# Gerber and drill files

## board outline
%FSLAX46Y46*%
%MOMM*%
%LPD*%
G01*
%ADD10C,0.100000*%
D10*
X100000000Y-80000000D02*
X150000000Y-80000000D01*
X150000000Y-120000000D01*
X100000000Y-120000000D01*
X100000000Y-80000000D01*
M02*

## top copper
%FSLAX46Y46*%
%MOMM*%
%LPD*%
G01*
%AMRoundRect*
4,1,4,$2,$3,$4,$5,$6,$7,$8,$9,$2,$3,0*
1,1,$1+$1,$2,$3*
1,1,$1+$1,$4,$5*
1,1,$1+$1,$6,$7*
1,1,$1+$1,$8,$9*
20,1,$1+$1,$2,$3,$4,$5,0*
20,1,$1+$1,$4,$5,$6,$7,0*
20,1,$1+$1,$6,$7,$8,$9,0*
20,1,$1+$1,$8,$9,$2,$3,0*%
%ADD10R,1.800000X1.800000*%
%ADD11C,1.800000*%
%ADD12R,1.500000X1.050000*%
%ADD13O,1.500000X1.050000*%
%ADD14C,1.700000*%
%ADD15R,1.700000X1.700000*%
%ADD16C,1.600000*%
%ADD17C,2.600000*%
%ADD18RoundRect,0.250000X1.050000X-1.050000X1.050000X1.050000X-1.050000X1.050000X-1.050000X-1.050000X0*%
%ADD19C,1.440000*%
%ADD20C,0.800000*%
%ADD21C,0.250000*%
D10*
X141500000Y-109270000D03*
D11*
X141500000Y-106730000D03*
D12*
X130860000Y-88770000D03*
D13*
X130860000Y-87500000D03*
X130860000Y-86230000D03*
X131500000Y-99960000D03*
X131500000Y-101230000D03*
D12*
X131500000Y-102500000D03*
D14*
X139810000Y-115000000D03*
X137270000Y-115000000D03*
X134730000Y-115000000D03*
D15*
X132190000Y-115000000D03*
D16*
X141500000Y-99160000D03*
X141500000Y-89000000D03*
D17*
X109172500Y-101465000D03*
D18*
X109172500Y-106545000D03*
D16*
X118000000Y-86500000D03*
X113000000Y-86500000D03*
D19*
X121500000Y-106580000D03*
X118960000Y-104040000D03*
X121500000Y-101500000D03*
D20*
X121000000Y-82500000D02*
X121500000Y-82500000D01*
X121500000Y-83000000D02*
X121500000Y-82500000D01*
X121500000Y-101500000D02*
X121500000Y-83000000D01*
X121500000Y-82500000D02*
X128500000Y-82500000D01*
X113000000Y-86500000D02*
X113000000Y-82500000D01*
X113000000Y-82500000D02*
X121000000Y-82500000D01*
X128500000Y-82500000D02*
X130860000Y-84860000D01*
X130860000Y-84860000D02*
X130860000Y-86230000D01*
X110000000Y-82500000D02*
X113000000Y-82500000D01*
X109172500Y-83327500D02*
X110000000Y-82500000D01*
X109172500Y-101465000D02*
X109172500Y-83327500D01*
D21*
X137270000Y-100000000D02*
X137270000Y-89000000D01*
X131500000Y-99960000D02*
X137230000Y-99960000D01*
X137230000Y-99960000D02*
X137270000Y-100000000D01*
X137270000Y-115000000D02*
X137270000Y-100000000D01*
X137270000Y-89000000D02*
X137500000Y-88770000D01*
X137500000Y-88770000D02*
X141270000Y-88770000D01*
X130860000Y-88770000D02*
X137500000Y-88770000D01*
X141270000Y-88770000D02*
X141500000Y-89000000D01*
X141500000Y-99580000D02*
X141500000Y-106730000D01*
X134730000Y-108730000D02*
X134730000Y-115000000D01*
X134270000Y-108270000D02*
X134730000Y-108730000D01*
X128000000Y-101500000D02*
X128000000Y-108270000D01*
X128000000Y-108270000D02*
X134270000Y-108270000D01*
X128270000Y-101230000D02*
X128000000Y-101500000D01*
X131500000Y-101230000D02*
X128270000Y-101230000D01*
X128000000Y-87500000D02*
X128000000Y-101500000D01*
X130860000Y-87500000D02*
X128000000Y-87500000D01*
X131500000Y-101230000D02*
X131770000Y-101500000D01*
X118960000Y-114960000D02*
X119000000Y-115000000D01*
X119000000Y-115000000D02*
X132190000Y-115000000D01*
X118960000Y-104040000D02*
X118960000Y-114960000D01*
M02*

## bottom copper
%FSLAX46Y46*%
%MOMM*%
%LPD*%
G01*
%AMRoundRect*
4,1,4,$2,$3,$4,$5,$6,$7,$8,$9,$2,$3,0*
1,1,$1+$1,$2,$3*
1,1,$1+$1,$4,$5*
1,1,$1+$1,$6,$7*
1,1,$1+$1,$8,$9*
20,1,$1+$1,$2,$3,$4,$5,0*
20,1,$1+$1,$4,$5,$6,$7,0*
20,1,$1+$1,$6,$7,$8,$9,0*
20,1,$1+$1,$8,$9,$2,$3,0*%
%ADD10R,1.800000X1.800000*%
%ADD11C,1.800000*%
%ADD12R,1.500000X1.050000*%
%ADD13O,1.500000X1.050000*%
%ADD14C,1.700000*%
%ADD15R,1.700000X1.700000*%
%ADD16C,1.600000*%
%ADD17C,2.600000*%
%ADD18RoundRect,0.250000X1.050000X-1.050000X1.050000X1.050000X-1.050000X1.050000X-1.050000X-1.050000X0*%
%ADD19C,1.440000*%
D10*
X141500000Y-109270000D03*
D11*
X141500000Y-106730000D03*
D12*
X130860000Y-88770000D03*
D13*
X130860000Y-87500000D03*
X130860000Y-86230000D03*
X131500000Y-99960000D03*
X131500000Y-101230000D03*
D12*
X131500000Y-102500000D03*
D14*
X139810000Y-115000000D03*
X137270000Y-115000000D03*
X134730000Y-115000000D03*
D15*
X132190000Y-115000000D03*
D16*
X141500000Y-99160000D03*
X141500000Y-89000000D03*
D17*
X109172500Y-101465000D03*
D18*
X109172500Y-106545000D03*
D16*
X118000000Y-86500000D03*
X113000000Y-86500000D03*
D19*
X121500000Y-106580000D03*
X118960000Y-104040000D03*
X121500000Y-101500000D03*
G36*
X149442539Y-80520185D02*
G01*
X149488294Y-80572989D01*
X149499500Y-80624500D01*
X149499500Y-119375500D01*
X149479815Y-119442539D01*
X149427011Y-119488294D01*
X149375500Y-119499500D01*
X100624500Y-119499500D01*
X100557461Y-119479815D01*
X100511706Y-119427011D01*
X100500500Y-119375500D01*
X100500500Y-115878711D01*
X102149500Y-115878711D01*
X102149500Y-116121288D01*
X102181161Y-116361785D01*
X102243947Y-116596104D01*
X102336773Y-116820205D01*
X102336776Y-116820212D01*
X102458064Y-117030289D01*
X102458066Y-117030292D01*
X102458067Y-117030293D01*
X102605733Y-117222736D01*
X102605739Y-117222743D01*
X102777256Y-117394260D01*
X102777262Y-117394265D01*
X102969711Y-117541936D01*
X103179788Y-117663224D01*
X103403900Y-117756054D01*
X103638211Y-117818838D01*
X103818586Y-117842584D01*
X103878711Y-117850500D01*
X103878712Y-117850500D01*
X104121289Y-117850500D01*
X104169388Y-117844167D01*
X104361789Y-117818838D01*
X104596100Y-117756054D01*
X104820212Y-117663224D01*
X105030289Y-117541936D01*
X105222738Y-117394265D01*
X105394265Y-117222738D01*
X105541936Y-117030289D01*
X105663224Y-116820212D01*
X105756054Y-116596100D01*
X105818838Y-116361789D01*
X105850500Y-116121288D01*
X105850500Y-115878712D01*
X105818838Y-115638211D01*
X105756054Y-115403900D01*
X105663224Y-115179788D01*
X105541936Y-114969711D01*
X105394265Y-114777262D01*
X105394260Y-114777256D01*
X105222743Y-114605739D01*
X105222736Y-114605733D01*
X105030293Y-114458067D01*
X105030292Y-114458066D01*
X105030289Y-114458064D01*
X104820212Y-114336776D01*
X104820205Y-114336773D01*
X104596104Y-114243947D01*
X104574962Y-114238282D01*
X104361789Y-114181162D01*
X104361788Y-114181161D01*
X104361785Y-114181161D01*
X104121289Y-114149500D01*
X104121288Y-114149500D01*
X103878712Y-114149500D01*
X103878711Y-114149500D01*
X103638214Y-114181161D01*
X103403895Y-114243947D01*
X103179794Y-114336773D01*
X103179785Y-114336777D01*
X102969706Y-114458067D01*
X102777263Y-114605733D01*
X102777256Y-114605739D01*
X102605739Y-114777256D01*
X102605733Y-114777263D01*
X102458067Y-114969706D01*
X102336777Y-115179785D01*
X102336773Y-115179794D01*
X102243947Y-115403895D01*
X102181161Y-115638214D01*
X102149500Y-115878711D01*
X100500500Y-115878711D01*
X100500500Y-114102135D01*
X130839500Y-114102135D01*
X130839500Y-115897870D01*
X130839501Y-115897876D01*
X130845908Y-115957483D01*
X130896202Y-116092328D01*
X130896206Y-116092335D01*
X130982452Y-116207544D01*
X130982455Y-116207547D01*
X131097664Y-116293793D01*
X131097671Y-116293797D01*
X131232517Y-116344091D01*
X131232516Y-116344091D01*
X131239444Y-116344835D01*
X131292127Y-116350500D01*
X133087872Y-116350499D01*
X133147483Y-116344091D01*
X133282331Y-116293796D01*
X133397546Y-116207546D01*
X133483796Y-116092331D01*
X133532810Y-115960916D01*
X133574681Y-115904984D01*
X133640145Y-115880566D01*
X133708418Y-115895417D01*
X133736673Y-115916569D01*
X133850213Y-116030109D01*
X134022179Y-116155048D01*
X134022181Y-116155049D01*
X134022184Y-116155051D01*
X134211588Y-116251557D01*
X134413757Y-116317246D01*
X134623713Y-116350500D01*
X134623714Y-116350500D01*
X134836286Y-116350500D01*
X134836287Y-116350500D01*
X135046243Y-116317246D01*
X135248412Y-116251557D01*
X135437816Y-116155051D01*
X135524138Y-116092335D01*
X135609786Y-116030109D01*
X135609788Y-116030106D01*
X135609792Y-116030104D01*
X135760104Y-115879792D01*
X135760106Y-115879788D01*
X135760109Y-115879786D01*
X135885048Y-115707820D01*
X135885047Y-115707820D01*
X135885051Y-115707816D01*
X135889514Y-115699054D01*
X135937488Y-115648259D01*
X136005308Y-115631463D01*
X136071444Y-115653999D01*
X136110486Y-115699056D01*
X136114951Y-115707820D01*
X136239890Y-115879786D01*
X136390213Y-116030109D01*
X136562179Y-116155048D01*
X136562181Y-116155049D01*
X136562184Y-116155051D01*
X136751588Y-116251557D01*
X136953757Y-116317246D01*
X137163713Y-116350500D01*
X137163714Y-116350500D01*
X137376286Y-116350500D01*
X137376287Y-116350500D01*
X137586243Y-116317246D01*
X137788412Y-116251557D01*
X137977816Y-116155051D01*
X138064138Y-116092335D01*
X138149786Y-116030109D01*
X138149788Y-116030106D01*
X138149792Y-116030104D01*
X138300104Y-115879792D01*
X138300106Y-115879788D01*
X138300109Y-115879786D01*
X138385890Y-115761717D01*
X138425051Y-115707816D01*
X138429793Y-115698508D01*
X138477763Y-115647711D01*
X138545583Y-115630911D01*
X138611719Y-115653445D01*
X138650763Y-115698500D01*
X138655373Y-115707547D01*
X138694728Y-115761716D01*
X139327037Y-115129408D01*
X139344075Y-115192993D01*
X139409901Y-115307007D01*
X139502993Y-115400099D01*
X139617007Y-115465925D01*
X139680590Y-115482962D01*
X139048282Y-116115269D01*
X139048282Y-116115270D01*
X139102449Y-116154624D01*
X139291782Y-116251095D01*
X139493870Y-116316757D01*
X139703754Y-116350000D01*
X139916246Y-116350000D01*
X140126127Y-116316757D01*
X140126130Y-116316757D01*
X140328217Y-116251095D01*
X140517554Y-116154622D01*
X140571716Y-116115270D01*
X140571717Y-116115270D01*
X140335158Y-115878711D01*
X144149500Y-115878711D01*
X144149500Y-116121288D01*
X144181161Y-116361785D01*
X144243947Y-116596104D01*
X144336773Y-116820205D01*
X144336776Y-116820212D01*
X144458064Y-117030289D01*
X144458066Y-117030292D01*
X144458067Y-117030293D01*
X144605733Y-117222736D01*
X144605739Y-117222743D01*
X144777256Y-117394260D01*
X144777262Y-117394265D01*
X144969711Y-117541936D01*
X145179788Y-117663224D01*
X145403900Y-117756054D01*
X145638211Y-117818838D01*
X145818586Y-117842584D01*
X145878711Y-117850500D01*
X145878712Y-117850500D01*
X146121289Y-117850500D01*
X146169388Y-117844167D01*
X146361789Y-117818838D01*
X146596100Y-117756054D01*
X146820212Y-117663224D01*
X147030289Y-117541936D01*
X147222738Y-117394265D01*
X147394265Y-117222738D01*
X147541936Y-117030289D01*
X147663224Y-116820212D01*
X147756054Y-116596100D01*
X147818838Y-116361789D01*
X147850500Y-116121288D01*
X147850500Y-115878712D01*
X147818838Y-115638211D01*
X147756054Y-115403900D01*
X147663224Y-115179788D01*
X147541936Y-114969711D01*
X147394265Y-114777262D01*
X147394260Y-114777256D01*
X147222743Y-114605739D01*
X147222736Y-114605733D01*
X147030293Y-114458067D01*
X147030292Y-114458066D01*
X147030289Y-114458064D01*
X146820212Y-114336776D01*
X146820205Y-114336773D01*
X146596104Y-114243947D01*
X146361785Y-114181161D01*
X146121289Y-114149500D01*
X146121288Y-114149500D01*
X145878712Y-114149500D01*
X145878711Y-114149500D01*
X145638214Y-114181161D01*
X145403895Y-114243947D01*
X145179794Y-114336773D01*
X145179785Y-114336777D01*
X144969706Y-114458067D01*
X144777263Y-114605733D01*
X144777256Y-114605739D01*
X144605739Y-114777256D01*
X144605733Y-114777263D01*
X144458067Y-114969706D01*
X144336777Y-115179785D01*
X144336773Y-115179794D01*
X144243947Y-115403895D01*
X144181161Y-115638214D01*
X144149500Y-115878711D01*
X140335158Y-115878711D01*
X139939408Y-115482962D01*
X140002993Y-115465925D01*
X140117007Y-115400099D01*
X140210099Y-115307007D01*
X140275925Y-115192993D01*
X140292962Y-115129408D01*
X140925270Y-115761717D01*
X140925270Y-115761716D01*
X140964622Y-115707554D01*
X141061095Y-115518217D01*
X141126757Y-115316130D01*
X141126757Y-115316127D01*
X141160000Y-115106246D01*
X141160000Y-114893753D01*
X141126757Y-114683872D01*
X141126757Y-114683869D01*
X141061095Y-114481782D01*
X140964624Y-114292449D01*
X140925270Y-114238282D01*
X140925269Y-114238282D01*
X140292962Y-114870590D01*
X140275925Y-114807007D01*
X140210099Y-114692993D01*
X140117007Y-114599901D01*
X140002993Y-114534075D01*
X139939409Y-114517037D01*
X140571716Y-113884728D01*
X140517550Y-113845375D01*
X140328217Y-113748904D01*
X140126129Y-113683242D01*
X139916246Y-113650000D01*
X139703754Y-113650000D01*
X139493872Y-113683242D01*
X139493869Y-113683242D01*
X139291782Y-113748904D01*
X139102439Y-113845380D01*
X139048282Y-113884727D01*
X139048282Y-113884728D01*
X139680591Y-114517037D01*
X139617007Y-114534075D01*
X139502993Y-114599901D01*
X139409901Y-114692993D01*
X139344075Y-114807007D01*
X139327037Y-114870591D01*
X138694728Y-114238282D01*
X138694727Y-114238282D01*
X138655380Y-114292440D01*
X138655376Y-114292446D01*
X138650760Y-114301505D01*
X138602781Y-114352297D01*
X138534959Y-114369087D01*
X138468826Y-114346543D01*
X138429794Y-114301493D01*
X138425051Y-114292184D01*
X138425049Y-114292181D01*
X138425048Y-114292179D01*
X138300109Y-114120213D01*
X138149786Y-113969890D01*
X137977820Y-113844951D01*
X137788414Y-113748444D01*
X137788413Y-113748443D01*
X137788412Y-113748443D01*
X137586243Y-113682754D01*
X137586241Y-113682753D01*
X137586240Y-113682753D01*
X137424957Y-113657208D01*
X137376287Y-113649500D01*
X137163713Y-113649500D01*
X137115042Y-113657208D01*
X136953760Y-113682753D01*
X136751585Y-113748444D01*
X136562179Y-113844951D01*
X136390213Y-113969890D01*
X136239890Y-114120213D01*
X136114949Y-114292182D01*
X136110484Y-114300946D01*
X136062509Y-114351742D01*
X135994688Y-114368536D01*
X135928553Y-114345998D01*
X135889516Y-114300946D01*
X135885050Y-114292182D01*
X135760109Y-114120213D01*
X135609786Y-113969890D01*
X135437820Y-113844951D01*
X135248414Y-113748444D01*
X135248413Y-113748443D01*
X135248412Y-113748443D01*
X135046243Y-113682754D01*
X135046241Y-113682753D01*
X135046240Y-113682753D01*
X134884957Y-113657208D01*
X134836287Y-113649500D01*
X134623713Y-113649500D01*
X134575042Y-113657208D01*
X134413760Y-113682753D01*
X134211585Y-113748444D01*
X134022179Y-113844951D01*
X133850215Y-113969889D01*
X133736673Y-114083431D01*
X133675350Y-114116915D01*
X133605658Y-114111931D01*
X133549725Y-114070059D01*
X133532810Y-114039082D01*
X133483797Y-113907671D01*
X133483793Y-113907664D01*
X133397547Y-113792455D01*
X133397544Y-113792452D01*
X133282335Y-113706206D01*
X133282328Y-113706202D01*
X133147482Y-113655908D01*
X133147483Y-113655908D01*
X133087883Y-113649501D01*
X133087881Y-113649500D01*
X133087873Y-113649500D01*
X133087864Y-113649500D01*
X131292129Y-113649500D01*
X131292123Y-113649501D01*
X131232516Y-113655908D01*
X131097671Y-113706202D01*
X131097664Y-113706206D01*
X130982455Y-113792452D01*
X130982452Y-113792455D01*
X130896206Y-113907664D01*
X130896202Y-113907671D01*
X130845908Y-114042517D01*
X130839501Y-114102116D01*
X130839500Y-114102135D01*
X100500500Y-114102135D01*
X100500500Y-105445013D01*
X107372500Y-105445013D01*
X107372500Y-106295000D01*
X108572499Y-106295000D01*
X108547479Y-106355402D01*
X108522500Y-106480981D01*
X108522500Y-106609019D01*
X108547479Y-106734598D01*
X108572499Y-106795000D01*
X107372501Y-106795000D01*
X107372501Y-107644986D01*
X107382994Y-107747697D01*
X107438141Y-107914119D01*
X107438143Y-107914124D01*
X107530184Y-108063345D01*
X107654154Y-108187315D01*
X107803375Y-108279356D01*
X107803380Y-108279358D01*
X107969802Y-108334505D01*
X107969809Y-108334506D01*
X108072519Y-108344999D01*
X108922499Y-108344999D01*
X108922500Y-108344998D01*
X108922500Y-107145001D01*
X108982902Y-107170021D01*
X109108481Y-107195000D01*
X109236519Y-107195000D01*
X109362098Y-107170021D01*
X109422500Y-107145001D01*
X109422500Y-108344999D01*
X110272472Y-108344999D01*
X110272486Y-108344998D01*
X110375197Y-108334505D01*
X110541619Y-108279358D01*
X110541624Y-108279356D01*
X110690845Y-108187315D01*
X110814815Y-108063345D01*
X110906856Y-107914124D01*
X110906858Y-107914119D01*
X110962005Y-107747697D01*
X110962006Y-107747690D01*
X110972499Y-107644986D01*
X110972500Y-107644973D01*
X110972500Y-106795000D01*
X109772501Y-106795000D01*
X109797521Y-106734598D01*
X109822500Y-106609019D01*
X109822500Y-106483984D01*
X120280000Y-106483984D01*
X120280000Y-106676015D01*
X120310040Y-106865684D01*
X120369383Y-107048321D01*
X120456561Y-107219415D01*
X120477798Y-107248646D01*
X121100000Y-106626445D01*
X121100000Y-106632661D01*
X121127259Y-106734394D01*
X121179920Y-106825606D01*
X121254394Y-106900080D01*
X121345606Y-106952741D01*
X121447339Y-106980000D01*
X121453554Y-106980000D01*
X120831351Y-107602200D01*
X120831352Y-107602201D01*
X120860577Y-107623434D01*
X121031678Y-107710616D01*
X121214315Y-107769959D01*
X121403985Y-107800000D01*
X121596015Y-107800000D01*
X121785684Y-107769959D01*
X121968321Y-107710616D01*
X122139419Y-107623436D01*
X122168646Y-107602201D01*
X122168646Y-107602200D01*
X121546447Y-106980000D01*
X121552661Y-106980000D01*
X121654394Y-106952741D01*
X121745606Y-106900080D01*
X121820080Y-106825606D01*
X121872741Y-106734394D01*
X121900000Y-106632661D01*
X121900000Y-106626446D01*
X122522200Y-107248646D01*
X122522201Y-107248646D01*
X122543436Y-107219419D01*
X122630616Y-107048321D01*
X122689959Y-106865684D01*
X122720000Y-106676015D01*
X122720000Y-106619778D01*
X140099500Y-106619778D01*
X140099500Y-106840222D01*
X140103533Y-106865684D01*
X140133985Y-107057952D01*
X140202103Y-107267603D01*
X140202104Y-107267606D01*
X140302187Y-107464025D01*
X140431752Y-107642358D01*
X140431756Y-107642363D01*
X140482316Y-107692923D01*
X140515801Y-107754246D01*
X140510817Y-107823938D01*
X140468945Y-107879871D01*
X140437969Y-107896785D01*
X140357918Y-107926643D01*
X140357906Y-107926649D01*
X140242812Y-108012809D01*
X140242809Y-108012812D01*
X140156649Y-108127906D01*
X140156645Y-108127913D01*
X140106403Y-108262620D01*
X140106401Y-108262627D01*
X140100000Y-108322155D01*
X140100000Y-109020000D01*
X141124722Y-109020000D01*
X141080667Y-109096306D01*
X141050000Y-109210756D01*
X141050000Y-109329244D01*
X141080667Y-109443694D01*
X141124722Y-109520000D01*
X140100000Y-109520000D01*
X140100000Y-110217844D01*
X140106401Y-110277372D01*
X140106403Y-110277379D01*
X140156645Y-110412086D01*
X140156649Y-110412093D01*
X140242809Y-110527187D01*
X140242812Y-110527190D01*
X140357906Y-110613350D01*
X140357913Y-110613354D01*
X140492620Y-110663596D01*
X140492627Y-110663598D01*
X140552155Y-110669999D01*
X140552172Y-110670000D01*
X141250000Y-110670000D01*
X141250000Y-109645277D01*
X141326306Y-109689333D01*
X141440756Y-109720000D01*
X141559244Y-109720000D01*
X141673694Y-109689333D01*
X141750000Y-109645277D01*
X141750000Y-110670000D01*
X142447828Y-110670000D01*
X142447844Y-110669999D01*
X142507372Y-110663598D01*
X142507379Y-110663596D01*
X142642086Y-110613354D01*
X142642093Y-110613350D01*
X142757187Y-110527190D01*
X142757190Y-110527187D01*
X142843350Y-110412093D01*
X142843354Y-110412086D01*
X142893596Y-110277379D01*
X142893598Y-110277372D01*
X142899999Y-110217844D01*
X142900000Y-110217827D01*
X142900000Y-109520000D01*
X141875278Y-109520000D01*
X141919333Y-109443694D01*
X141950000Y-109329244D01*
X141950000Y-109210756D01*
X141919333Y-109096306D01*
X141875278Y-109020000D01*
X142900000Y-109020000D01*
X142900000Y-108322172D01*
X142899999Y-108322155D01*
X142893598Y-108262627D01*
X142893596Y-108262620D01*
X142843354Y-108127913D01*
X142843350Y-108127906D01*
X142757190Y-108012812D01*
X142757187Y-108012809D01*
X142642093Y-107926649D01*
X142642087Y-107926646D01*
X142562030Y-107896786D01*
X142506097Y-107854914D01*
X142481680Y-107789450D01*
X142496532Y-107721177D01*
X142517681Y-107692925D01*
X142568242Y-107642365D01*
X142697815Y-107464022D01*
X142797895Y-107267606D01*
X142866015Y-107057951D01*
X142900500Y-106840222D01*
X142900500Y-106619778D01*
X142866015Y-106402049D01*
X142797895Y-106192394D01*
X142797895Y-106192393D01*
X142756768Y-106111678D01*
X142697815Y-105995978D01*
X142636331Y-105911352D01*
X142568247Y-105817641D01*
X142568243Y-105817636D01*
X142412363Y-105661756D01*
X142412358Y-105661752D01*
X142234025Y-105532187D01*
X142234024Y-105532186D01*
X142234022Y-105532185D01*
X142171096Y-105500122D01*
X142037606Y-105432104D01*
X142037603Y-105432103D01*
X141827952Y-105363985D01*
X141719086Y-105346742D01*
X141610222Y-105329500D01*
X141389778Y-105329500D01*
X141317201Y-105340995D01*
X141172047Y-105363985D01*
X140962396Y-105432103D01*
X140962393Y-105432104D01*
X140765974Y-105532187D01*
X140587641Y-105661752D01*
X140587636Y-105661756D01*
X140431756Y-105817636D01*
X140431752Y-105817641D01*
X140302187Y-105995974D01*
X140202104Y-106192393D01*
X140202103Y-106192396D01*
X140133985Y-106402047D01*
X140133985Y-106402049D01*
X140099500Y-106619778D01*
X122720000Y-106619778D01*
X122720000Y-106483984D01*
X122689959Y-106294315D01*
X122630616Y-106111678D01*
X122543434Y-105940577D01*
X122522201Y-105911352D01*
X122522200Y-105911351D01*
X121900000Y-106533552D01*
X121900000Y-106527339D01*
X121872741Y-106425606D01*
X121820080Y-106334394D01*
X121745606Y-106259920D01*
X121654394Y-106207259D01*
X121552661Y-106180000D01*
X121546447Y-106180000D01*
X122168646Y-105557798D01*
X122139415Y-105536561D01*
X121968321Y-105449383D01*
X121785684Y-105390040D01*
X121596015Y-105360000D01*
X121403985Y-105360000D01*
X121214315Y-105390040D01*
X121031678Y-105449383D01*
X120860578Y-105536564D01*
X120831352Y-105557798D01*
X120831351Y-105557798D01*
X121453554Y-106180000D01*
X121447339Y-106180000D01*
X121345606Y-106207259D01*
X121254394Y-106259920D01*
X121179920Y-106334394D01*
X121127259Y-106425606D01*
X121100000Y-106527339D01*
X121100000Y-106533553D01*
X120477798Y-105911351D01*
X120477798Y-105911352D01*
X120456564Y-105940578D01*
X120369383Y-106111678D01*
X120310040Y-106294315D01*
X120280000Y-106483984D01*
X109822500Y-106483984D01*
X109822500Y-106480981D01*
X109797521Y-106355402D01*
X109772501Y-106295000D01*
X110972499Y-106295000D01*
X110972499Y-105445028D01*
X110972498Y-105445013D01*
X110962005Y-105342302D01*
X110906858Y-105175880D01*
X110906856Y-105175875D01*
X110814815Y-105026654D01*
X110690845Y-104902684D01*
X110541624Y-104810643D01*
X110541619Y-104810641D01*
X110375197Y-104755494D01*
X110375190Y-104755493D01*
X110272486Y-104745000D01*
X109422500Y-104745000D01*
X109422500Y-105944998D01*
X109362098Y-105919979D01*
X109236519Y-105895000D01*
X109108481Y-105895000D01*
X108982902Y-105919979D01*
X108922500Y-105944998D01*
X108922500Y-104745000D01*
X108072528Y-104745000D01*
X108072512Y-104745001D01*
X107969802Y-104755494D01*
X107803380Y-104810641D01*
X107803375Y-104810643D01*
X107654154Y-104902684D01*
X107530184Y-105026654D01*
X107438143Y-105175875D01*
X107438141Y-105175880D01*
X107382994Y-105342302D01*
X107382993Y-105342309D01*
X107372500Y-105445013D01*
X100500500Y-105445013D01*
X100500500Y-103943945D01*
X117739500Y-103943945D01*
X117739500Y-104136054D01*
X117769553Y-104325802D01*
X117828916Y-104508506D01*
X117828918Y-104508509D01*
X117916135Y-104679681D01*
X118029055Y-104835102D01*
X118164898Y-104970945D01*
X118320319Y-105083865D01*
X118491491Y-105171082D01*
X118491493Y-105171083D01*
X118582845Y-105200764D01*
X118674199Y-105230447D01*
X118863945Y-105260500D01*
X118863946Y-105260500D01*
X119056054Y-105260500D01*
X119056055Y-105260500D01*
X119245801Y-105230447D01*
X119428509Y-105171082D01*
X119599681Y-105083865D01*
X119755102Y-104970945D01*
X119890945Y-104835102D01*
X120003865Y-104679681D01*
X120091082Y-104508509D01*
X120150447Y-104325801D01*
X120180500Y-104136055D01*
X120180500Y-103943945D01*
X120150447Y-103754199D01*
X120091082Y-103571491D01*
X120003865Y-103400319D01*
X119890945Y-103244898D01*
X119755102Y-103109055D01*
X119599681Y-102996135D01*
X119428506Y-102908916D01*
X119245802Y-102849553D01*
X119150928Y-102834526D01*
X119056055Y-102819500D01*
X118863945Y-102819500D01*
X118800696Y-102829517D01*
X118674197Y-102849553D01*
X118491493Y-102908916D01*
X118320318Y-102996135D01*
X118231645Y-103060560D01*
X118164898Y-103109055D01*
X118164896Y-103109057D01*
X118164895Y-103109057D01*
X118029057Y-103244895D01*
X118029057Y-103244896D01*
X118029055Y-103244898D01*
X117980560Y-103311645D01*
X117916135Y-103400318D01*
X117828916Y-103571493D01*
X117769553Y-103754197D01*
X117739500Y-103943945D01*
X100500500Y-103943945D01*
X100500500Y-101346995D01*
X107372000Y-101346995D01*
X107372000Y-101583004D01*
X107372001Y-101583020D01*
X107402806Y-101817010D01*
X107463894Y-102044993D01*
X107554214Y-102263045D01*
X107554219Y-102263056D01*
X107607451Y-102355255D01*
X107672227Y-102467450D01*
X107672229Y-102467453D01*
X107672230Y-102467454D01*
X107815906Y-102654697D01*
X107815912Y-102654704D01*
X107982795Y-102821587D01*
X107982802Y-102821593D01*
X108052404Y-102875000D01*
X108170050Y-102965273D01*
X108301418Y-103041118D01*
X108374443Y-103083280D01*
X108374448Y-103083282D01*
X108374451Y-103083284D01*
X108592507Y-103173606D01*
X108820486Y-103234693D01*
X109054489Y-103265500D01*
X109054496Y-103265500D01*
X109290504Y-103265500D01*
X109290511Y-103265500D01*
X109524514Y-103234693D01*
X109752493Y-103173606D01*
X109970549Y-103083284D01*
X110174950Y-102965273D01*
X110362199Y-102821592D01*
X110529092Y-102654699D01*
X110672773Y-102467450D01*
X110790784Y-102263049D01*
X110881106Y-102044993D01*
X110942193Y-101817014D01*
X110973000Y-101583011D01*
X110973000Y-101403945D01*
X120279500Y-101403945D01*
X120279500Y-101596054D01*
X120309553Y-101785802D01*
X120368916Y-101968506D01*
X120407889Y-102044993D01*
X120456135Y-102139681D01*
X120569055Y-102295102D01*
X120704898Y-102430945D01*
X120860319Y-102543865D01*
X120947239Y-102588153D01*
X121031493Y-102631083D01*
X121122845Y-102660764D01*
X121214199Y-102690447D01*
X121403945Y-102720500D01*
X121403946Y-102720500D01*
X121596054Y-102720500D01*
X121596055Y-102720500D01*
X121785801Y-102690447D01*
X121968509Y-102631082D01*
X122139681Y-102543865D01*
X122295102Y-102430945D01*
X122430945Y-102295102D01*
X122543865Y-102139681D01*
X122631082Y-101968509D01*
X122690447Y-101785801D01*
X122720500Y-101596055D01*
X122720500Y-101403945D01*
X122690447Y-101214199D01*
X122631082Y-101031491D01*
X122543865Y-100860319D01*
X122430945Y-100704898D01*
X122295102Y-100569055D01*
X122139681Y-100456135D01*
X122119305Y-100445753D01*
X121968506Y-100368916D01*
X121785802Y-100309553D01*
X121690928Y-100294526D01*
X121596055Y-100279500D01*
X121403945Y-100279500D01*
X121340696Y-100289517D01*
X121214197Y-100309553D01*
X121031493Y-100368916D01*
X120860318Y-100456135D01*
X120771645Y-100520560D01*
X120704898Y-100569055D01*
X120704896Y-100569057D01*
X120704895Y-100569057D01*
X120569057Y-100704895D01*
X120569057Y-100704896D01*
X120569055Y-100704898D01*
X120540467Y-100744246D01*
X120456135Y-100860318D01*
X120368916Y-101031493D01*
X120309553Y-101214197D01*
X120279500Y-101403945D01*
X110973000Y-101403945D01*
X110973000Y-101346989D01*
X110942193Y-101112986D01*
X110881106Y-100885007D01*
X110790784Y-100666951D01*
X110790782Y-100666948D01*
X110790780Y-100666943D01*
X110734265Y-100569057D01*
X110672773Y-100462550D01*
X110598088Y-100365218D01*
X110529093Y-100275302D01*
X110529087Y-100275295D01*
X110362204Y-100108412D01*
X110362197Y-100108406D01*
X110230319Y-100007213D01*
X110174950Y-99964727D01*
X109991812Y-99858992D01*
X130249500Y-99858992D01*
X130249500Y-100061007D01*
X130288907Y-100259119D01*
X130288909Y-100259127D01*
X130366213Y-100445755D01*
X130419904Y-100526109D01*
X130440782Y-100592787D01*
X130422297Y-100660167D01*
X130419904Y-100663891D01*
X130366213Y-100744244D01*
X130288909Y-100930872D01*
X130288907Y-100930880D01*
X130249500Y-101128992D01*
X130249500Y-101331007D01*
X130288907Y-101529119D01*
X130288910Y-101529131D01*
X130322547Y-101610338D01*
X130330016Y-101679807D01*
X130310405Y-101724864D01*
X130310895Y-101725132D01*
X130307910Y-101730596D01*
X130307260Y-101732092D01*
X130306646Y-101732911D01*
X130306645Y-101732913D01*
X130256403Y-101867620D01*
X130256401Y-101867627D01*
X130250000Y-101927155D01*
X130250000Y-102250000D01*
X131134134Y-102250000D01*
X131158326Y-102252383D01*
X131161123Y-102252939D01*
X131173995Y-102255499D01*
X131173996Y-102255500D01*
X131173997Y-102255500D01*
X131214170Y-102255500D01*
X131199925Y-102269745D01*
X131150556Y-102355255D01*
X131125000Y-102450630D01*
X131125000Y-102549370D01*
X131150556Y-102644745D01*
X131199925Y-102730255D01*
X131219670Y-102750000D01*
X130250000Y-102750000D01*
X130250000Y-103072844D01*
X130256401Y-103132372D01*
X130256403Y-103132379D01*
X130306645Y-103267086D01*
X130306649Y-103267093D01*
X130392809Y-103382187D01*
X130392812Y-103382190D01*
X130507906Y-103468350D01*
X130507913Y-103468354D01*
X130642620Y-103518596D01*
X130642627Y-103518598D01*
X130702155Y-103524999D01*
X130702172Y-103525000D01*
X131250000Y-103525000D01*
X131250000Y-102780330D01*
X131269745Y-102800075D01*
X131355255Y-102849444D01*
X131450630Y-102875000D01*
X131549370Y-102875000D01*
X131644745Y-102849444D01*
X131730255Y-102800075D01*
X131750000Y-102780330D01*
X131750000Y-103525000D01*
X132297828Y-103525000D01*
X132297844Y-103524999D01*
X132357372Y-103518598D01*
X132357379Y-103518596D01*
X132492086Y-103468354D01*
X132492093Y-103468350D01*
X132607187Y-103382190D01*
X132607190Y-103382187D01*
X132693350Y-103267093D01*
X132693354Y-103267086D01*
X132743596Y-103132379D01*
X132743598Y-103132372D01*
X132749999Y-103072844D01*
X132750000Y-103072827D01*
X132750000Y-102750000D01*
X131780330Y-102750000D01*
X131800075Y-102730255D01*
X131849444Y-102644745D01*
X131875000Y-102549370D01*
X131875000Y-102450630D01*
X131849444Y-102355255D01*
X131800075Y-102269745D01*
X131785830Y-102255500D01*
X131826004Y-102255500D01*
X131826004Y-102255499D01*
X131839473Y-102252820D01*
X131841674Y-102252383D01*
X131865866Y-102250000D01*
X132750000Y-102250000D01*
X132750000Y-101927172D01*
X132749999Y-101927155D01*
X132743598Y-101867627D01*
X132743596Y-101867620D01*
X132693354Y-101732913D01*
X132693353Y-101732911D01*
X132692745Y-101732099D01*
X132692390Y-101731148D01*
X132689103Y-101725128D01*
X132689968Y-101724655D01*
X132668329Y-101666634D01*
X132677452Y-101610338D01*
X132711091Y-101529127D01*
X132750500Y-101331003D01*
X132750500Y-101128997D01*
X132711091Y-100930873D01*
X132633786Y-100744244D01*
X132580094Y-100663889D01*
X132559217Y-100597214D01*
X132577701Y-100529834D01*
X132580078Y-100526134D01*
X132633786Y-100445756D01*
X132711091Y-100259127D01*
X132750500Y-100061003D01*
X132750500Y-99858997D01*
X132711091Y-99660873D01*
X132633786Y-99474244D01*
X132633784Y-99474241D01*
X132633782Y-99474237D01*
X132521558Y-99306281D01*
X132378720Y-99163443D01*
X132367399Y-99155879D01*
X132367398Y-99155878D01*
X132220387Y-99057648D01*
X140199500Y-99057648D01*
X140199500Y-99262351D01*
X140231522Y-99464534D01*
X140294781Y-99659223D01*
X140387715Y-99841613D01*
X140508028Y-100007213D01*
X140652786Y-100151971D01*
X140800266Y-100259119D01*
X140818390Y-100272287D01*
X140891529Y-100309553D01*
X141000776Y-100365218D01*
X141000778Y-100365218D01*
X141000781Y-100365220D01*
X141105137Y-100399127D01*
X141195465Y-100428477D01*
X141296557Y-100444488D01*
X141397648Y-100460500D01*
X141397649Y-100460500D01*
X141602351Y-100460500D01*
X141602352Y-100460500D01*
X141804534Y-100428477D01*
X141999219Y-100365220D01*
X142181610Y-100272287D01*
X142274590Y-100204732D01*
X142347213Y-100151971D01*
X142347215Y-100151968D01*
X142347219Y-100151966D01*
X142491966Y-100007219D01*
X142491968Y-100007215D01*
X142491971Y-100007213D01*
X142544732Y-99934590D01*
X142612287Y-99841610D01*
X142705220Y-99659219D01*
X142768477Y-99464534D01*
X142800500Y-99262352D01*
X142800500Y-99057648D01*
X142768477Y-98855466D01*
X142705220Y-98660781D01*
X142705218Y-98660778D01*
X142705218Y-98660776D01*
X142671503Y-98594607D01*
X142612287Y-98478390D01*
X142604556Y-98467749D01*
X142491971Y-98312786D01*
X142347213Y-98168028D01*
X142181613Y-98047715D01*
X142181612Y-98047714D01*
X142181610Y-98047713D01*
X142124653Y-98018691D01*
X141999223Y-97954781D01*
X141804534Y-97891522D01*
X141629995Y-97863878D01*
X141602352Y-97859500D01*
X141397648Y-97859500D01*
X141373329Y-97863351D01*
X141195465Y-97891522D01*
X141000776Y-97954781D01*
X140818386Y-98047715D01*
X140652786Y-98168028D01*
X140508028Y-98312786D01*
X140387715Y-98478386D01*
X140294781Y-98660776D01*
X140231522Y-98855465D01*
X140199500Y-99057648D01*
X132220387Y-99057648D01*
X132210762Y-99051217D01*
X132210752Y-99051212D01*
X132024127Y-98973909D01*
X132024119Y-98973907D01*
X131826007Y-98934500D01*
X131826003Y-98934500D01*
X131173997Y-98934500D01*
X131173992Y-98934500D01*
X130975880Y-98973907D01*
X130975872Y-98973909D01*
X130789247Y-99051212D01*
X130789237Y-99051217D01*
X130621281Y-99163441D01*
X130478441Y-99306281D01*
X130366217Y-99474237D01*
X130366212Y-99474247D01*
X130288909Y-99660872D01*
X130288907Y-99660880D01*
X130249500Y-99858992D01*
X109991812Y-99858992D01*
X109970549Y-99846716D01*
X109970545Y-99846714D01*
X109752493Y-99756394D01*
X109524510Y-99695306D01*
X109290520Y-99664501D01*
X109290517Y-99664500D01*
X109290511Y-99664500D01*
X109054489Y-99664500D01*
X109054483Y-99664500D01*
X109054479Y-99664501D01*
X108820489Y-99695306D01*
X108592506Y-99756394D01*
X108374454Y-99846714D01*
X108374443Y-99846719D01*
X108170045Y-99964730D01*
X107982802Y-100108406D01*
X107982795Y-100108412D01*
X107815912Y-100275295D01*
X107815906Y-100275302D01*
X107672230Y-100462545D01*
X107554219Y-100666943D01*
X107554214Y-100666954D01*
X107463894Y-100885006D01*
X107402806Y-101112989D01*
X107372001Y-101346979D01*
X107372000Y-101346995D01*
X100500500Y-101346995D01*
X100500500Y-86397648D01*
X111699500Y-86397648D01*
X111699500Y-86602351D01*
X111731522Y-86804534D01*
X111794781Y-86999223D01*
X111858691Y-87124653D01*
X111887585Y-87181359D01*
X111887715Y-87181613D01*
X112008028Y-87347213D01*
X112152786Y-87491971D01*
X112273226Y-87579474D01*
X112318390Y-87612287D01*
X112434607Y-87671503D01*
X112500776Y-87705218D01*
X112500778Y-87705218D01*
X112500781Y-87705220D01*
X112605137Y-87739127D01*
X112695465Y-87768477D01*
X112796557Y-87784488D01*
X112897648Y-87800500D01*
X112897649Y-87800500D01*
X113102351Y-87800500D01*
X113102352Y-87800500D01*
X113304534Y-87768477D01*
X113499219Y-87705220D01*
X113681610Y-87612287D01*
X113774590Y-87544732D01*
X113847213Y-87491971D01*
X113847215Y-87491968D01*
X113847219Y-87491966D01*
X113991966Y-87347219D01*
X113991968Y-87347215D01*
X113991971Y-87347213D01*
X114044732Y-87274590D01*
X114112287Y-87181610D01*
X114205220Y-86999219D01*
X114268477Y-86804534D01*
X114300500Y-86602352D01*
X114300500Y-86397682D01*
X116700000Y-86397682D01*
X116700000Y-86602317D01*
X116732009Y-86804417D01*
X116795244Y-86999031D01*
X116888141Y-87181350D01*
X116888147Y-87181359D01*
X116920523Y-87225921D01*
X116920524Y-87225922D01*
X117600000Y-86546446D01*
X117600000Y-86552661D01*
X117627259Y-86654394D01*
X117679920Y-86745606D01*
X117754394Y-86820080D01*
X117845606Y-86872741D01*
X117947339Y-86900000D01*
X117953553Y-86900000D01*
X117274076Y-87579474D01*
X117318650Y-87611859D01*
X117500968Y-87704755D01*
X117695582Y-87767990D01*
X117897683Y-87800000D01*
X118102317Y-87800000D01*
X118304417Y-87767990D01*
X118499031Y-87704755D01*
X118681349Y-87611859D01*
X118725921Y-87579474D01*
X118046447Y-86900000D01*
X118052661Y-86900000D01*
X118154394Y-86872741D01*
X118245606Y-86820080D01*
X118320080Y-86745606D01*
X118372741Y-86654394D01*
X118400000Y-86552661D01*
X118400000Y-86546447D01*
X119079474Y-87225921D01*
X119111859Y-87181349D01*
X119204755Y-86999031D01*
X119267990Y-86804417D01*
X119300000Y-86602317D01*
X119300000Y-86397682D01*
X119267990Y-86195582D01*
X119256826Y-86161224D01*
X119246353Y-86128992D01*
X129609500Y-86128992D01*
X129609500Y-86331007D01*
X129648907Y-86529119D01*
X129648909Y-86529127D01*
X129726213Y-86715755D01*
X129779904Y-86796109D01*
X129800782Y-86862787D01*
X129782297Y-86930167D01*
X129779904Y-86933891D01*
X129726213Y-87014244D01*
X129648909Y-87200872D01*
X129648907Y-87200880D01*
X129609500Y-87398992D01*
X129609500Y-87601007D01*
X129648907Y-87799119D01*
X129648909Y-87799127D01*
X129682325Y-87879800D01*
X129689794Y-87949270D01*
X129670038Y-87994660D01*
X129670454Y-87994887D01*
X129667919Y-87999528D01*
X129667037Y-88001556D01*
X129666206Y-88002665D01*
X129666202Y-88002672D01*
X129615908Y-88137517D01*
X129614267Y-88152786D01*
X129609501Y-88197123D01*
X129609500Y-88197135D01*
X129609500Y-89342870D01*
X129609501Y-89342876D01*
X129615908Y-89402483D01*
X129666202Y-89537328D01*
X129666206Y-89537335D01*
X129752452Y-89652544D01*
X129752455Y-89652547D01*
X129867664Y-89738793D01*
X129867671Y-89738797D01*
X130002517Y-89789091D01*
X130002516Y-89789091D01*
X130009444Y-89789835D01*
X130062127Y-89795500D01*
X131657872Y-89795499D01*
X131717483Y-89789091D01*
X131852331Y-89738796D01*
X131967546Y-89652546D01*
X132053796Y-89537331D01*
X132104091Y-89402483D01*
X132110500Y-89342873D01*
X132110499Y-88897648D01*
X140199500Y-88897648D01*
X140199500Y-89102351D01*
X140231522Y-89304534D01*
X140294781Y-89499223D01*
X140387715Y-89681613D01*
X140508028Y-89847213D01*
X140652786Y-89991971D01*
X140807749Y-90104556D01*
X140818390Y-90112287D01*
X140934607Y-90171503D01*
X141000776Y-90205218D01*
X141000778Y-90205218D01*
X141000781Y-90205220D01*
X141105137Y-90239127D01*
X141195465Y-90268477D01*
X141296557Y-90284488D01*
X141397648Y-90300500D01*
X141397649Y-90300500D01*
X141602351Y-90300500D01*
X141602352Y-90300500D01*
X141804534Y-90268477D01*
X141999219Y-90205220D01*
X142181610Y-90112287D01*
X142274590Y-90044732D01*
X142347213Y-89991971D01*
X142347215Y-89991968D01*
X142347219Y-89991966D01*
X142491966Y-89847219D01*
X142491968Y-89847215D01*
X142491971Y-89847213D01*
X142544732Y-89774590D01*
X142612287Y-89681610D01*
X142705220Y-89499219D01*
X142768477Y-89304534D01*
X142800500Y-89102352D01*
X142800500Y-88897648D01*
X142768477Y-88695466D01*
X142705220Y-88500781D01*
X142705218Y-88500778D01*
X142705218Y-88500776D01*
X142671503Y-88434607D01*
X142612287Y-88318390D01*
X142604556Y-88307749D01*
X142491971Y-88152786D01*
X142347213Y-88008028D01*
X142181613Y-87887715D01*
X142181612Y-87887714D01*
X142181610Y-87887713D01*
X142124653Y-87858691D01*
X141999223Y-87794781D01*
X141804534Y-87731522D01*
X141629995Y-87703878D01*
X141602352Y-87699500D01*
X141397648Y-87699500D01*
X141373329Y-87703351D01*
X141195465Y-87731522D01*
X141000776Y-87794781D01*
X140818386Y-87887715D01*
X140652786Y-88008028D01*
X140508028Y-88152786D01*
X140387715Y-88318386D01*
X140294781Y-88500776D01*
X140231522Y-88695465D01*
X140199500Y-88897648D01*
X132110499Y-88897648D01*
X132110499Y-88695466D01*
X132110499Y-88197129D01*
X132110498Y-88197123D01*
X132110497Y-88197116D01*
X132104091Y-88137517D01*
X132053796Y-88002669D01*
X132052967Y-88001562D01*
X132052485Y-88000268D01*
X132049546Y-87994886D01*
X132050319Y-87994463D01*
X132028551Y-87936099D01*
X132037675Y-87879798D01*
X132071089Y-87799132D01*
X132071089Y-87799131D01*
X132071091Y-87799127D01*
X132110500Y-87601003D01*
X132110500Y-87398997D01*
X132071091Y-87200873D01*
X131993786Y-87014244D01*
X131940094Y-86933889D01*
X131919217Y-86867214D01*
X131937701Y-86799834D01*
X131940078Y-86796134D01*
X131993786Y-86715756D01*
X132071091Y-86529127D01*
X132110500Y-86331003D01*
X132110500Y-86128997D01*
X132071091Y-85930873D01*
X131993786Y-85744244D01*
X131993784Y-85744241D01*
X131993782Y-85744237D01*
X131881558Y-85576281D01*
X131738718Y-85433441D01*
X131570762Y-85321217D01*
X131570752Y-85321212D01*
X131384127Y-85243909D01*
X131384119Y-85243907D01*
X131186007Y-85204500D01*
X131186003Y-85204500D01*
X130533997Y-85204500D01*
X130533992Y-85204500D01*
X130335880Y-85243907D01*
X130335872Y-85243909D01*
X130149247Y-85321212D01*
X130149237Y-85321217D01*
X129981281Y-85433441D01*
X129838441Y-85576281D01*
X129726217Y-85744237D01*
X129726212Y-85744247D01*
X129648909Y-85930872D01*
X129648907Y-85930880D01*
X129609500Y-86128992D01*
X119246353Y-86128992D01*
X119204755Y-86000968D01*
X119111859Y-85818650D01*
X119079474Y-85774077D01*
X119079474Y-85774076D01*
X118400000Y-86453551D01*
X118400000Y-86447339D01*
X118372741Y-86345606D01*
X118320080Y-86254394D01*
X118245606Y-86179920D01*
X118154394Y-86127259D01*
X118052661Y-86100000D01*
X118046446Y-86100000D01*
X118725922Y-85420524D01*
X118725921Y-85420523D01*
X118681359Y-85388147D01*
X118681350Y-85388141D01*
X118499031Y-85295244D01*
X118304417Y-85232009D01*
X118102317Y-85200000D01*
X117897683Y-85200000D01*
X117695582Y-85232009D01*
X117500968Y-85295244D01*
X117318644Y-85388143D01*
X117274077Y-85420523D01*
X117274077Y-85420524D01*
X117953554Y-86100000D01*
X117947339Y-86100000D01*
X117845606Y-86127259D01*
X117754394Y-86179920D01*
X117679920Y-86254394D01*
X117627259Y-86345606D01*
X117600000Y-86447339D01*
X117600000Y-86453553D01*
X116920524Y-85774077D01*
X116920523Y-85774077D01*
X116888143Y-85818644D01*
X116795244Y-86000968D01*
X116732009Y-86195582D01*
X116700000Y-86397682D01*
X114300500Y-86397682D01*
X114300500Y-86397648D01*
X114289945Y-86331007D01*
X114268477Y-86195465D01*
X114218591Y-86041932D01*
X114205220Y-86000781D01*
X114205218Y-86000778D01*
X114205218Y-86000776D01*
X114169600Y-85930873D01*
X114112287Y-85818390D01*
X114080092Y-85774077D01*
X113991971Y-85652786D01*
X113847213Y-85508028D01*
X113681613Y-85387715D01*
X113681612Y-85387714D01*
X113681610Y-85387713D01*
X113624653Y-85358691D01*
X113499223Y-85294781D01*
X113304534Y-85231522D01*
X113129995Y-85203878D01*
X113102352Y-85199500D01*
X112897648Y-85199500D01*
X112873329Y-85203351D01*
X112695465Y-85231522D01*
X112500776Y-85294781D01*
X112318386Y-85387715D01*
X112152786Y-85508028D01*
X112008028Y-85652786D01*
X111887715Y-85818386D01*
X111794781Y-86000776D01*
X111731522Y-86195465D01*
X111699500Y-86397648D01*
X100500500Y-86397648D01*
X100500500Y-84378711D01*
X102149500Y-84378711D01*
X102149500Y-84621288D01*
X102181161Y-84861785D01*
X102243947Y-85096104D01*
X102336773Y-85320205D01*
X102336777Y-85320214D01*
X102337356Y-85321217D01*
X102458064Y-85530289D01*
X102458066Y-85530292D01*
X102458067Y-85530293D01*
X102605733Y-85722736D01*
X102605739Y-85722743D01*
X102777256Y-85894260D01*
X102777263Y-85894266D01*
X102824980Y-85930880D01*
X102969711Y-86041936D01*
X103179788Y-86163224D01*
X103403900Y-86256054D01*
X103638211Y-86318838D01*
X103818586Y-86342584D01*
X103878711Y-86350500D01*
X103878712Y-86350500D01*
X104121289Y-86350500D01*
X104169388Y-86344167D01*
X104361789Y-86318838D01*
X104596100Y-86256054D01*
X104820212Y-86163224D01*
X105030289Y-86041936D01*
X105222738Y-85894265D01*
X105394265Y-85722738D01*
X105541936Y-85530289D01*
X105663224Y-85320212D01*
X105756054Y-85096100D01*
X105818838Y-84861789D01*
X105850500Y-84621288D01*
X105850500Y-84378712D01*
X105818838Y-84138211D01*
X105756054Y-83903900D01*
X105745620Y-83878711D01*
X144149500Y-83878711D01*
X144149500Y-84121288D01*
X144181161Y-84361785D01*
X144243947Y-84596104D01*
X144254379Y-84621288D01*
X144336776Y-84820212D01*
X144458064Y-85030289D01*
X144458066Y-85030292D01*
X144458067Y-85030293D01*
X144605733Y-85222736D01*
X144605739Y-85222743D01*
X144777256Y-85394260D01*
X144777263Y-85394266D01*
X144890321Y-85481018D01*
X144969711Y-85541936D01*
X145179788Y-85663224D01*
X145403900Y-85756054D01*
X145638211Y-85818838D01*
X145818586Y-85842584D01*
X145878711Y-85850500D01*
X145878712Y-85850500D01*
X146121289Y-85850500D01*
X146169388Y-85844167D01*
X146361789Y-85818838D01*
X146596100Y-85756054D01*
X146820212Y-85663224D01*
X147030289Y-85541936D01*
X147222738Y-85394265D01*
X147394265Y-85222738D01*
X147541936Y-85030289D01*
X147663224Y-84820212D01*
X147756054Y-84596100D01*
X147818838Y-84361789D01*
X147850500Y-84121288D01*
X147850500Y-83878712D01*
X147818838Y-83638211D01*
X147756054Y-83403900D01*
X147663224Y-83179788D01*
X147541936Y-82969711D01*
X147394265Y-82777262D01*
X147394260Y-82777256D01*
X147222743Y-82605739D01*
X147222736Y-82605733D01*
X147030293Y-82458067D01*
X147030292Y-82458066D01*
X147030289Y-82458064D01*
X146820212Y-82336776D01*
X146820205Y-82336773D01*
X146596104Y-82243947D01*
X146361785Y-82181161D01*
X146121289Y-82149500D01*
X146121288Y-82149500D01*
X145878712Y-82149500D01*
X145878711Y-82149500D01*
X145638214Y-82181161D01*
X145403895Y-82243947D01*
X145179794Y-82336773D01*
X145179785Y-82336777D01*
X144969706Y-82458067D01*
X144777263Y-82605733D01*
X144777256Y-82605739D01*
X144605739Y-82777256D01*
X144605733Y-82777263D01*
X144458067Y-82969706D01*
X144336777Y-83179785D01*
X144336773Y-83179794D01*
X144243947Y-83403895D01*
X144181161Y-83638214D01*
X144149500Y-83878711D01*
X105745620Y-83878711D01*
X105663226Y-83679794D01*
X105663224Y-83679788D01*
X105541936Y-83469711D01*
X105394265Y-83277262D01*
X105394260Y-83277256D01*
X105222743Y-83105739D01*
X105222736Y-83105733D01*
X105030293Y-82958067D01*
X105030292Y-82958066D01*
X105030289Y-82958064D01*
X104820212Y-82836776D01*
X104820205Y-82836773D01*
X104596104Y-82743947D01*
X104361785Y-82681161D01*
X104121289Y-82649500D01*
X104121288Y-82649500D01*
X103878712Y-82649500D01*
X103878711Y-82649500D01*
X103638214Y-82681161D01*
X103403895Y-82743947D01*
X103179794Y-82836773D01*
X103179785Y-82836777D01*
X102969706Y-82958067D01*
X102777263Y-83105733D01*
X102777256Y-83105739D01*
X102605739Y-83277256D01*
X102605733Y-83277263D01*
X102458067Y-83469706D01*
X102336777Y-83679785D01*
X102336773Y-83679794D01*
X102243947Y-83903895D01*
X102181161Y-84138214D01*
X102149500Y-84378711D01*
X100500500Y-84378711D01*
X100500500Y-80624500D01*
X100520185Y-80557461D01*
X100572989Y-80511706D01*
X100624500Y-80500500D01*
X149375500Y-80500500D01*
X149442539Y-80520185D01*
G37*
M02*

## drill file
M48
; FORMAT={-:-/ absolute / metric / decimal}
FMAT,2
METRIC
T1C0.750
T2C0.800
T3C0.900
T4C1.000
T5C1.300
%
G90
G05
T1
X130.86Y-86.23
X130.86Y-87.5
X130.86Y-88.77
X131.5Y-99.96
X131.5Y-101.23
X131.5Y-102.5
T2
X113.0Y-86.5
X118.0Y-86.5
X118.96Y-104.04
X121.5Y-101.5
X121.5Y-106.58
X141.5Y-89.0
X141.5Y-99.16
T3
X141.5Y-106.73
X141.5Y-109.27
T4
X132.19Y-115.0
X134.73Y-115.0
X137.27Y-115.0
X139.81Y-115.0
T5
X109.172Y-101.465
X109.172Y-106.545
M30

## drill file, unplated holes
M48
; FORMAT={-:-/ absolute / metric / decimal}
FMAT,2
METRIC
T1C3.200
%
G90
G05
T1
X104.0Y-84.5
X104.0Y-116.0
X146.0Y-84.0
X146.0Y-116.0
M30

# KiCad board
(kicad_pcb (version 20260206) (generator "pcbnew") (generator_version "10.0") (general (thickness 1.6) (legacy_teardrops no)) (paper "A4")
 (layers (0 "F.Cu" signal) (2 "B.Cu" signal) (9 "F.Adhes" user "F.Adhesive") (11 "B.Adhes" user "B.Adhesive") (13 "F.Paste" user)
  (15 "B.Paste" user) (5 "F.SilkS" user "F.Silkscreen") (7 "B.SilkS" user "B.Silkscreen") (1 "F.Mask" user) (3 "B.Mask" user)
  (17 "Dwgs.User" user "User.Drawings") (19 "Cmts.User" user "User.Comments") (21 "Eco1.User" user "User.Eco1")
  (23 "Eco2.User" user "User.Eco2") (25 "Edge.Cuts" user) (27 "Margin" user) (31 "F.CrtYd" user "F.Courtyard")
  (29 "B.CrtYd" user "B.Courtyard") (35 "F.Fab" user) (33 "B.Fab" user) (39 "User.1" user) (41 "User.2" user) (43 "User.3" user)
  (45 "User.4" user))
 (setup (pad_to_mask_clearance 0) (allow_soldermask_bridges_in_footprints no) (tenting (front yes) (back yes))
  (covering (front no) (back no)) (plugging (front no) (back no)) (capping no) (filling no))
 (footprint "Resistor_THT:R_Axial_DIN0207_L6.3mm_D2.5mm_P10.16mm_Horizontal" (layer "F.Cu") (at 141.5 89 -90)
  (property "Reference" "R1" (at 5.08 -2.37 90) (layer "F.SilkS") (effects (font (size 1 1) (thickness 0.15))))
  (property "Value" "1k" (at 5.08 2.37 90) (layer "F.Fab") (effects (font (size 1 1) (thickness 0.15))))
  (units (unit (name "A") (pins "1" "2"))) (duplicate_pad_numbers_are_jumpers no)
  (pad "1" thru_hole circle (at 0 0 270) (size 1.6 1.6) (drill 0.8) (layers "*.Cu" "*.Mask") (remove_unused_layers no) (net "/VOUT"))
  (pad "2" thru_hole circle (at 10.16 0 270) (size 1.6 1.6) (drill 0.8) (layers "*.Cu" "*.Mask") (remove_unused_layers no)
   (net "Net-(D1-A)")))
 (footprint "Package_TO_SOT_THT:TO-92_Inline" (layer "F.Cu") (at 131.5 102.5 90)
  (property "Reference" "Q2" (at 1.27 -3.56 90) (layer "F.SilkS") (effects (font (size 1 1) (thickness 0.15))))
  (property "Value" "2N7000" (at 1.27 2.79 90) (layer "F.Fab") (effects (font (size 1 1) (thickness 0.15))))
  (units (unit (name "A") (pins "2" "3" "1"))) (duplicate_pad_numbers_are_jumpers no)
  (pad "1" thru_hole rect (at 0 0 90) (size 1.05 1.5) (drill 0.75) (layers "*.Cu" "*.Mask") (remove_unused_layers no) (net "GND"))
  (pad "2" thru_hole oval (at 1.27 0 90) (size 1.05 1.5) (drill 0.75) (layers "*.Cu" "*.Mask") (remove_unused_layers no) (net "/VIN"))
  (pad "3" thru_hole oval (at 2.54 0 90) (size 1.05 1.5) (drill 0.75) (layers "*.Cu" "*.Mask") (remove_unused_layers no) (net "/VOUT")))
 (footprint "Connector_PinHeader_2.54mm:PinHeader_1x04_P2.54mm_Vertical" (layer "F.Cu") (at 132.19 115 90)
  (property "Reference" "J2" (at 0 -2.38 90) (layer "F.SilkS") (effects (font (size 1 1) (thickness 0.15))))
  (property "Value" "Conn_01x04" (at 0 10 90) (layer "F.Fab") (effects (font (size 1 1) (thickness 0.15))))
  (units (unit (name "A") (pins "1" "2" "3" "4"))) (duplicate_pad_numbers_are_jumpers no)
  (pad "1" thru_hole rect (at 0 0 90) (size 1.7 1.7) (drill 1) (layers "*.Cu" "*.Mask") (remove_unused_layers no) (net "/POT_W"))
  (pad "2" thru_hole circle (at 0 2.54 90) (size 1.7 1.7) (drill 1) (layers "*.Cu" "*.Mask") (remove_unused_layers no) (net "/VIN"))
  (pad "3" thru_hole circle (at 0 5.08 90) (size 1.7 1.7) (drill 1) (layers "*.Cu" "*.Mask") (remove_unused_layers no) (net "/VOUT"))
  (pad "4" thru_hole circle (at 0 7.62 90) (size 1.7 1.7) (drill 1) (layers "*.Cu" "*.Mask") (remove_unused_layers no) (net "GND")))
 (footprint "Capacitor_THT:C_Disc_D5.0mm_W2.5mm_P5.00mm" (layer "F.Cu") (at 113 86.5)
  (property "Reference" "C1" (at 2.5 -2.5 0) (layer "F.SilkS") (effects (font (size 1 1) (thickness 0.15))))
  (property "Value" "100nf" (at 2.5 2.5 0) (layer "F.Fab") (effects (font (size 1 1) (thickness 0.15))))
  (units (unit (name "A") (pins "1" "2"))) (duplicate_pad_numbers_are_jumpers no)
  (pad "1" thru_hole circle (at 0 0) (size 1.6 1.6) (drill 0.8) (layers "*.Cu" "*.Mask") (remove_unused_layers no) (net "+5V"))
  (pad "2" thru_hole circle (at 5 0) (size 1.6 1.6) (drill 0.8) (layers "*.Cu" "*.Mask") (remove_unused_layers no) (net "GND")))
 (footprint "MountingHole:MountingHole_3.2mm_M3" (layer "F.Cu") (at 146 116)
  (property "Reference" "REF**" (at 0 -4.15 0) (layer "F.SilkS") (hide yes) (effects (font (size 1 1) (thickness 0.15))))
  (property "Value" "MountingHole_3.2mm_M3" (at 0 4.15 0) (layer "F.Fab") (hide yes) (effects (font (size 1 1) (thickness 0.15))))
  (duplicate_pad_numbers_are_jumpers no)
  (pad "" np_thru_hole circle (at 0 0) (size 3.2 3.2) (drill 3.2) (layers "*.Cu" "*.Mask")))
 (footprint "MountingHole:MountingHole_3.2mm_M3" (layer "F.Cu") (at 104 84.5)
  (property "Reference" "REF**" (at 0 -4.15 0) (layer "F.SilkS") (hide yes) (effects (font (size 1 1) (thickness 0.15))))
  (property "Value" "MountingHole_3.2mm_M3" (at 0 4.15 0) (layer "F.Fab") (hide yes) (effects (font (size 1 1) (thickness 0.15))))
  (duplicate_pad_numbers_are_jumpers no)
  (pad "" np_thru_hole circle (at 0 0) (size 3.2 3.2) (drill 3.2) (layers "*.Cu" "*.Mask")))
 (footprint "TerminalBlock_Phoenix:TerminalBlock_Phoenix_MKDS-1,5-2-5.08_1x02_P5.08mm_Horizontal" (layer "F.Cu") (at 109.1725 106.545 90)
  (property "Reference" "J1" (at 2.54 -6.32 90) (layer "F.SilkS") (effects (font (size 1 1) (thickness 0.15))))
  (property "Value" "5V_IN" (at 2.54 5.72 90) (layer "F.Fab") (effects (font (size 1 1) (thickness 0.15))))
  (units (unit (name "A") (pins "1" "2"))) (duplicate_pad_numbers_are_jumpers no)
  (pad "1" thru_hole roundrect (at 0 0 90) (size 2.6 2.6) (drill 1.3) (layers "*.Cu" "*.Mask") (remove_unused_layers no)
   (roundrect_rratio 0.096154) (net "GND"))
  (pad "2" thru_hole circle (at 5.08 0 90) (size 2.6 2.6) (drill 1.3) (layers "*.Cu" "*.Mask") (remove_unused_layers no) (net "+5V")))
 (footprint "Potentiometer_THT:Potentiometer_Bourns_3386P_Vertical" (layer "F.Cu") (at 121.5 101.5 180)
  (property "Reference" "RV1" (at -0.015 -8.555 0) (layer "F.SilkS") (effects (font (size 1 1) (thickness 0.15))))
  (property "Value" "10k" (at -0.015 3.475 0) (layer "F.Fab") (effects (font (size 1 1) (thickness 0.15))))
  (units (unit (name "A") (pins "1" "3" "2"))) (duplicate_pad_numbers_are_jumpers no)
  (pad "1" thru_hole circle (at 0 0 180) (size 1.44 1.44) (drill 0.8) (layers "*.Cu" "*.Mask") (remove_unused_layers no) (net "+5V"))
  (pad "2" thru_hole circle (at 2.54 -2.54 180) (size 1.44 1.44) (drill 0.8) (layers "*.Cu" "*.Mask") (remove_unused_layers no)
   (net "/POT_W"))
  (pad "3" thru_hole circle (at 0 -5.08 180) (size 1.44 1.44) (drill 0.8) (layers "*.Cu" "*.Mask") (remove_unused_layers no) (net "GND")))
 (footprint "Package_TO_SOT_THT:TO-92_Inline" (layer "F.Cu") (at 130.86 88.77 90)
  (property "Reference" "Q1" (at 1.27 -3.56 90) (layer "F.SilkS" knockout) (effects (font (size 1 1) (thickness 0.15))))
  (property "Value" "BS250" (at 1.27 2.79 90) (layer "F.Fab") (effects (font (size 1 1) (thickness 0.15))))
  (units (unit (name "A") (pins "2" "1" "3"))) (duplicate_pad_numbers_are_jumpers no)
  (pad "1" thru_hole rect (at 0 0 90) (size 1.05 1.5) (drill 0.75) (layers "*.Cu" "*.Mask") (remove_unused_layers no) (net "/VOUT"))
  (pad "2" thru_hole oval (at 1.27 0 90) (size 1.05 1.5) (drill 0.75) (layers "*.Cu" "*.Mask") (remove_unused_layers no) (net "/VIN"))
  (pad "3" thru_hole oval (at 2.54 0 90) (size 1.05 1.5) (drill 0.75) (layers "*.Cu" "*.Mask") (remove_unused_layers no) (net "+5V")))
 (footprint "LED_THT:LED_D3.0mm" (layer "F.Cu") (at 141.5 109.27 90)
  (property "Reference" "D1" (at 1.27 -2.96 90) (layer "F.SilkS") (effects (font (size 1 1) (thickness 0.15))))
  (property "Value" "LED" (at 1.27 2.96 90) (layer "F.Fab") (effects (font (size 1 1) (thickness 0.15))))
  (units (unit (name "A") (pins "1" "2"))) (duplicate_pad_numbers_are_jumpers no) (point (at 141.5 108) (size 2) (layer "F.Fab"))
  (pad "1" thru_hole rect (at 0 0 90) (size 1.8 1.8) (drill 0.9) (layers "*.Cu" "*.Mask") (remove_unused_layers no) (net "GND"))
  (pad "2" thru_hole circle (at 2.54 0 90) (size 1.8 1.8) (drill 0.9) (layers "*.Cu" "*.Mask") (remove_unused_layers no) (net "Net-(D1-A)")))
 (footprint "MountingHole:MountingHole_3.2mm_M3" (layer "F.Cu") (at 146 84)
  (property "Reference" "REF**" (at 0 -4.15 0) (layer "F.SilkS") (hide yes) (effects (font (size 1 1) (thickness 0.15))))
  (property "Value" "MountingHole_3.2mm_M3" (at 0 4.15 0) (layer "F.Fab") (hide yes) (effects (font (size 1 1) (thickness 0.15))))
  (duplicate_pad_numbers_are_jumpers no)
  (pad "" np_thru_hole circle (at 0 0) (size 3.2 3.2) (drill 3.2) (layers "*.Cu" "*.Mask")))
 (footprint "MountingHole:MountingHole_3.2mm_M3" (layer "F.Cu") (at 104 116)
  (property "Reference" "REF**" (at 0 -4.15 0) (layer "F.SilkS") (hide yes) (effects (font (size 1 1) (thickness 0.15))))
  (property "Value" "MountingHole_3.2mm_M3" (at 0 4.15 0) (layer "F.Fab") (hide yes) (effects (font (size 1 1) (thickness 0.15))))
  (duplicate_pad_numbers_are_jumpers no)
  (pad "" np_thru_hole circle (at 0 0) (size 3.2 3.2) (drill 3.2) (layers "*.Cu" "*.Mask")))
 (gr_rect (start 100 80) (end 150 120) (stroke (width 0.1) (type default)) (fill no) (layer "Edge.Cuts"))
 (segment (start 137.23 99.96) (end 137.27 100) (width 0.25) (layer "F.Cu") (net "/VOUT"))
 (segment (start 131.5 99.96) (end 137.23 99.96) (width 0.25) (layer "F.Cu") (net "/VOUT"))
 (segment (start 137.5 88.77) (end 141.27 88.77) (width 0.25) (layer "F.Cu") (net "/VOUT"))
 (segment (start 130.86 88.77) (end 137.5 88.77) (width 0.25) (layer "F.Cu") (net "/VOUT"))
 (segment (start 137.27 115) (end 137.27 100) (width 0.25) (layer "F.Cu") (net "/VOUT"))
 (segment (start 141.27 88.77) (end 141.5 89) (width 0.25) (layer "F.Cu") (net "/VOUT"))
 (segment (start 137.27 100) (end 137.27 89) (width 0.25) (layer "F.Cu") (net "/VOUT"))
 (segment (start 137.27 89) (end 137.5 88.77) (width 0.25) (layer "F.Cu") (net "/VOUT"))
 (segment (start 141.5 99.58) (end 141.5 106.73) (width 0.25) (layer "F.Cu") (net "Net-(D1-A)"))
 (segment (start 128 87.5) (end 128 101.5) (width 0.25) (layer "F.Cu") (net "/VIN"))
 (segment (start 131.5 101.23) (end 131.77 101.5) (width 0.25) (layer "F.Cu") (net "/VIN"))
 (segment (start 134.27 108.27) (end 134.73 108.73) (width 0.25) (layer "F.Cu") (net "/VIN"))
 (segment (start 128.27 101.23) (end 128 101.5) (width 0.25) (layer "F.Cu") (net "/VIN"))
 (segment (start 128 101.5) (end 128 108.27) (width 0.25) (layer "F.Cu") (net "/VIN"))
 (segment (start 131.5 101.23) (end 128.27 101.23) (width 0.25) (layer "F.Cu") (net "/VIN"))
 (segment (start 134.73 108.73) (end 134.73 115) (width 0.25) (layer "F.Cu") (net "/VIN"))
 (segment (start 130.86 87.5) (end 128 87.5) (width 0.25) (layer "F.Cu") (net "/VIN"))
 (segment (start 128 108.27) (end 134.27 108.27) (width 0.25) (layer "F.Cu") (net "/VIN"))
 (segment (start 118.96 104.04) (end 118.96 114.96) (width 0.25) (layer "F.Cu") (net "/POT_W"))
 (segment (start 118.96 114.96) (end 119 115) (width 0.25) (layer "F.Cu") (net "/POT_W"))
 (segment (start 119 115) (end 132.19 115) (width 0.25) (layer "F.Cu") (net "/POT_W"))
 (segment (start 121.5 101.5) (end 121.5 83) (width 0.8) (layer "F.Cu") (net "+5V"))
 (segment (start 121.5 83) (end 121.5 82.5) (width 0.8) (layer "F.Cu") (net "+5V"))
 (segment (start 109.1725 101.465) (end 109.1725 83.3275) (width 0.8) (layer "F.Cu") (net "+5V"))
 (segment (start 109.1725 83.3275) (end 110 82.5) (width 0.8) (layer "F.Cu") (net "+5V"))
 (segment (start 128.5 82.5) (end 130.86 84.86) (width 0.8) (layer "F.Cu") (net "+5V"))
 (segment (start 130.86 84.86) (end 130.86 86.23) (width 0.8) (layer "F.Cu") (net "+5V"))
 (segment (start 113 86.5) (end 113 82.5) (width 0.8) (layer "F.Cu") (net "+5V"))
 (segment (start 110 82.5) (end 113 82.5) (width 0.8) (layer "F.Cu") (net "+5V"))
 (segment (start 113 82.5) (end 121 82.5) (width 0.8) (layer "F.Cu") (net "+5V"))
 (segment (start 121 82.5) (end 121.5 82.5) (width 0.8) (layer "F.Cu") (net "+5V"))
 (segment (start 121.5 82.5) (end 128.5 82.5) (width 0.8) (layer "F.Cu") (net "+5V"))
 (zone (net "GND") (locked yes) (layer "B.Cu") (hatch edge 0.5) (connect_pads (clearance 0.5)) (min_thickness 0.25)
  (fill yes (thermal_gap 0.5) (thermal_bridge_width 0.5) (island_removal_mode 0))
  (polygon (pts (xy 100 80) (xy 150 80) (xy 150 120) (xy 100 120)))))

